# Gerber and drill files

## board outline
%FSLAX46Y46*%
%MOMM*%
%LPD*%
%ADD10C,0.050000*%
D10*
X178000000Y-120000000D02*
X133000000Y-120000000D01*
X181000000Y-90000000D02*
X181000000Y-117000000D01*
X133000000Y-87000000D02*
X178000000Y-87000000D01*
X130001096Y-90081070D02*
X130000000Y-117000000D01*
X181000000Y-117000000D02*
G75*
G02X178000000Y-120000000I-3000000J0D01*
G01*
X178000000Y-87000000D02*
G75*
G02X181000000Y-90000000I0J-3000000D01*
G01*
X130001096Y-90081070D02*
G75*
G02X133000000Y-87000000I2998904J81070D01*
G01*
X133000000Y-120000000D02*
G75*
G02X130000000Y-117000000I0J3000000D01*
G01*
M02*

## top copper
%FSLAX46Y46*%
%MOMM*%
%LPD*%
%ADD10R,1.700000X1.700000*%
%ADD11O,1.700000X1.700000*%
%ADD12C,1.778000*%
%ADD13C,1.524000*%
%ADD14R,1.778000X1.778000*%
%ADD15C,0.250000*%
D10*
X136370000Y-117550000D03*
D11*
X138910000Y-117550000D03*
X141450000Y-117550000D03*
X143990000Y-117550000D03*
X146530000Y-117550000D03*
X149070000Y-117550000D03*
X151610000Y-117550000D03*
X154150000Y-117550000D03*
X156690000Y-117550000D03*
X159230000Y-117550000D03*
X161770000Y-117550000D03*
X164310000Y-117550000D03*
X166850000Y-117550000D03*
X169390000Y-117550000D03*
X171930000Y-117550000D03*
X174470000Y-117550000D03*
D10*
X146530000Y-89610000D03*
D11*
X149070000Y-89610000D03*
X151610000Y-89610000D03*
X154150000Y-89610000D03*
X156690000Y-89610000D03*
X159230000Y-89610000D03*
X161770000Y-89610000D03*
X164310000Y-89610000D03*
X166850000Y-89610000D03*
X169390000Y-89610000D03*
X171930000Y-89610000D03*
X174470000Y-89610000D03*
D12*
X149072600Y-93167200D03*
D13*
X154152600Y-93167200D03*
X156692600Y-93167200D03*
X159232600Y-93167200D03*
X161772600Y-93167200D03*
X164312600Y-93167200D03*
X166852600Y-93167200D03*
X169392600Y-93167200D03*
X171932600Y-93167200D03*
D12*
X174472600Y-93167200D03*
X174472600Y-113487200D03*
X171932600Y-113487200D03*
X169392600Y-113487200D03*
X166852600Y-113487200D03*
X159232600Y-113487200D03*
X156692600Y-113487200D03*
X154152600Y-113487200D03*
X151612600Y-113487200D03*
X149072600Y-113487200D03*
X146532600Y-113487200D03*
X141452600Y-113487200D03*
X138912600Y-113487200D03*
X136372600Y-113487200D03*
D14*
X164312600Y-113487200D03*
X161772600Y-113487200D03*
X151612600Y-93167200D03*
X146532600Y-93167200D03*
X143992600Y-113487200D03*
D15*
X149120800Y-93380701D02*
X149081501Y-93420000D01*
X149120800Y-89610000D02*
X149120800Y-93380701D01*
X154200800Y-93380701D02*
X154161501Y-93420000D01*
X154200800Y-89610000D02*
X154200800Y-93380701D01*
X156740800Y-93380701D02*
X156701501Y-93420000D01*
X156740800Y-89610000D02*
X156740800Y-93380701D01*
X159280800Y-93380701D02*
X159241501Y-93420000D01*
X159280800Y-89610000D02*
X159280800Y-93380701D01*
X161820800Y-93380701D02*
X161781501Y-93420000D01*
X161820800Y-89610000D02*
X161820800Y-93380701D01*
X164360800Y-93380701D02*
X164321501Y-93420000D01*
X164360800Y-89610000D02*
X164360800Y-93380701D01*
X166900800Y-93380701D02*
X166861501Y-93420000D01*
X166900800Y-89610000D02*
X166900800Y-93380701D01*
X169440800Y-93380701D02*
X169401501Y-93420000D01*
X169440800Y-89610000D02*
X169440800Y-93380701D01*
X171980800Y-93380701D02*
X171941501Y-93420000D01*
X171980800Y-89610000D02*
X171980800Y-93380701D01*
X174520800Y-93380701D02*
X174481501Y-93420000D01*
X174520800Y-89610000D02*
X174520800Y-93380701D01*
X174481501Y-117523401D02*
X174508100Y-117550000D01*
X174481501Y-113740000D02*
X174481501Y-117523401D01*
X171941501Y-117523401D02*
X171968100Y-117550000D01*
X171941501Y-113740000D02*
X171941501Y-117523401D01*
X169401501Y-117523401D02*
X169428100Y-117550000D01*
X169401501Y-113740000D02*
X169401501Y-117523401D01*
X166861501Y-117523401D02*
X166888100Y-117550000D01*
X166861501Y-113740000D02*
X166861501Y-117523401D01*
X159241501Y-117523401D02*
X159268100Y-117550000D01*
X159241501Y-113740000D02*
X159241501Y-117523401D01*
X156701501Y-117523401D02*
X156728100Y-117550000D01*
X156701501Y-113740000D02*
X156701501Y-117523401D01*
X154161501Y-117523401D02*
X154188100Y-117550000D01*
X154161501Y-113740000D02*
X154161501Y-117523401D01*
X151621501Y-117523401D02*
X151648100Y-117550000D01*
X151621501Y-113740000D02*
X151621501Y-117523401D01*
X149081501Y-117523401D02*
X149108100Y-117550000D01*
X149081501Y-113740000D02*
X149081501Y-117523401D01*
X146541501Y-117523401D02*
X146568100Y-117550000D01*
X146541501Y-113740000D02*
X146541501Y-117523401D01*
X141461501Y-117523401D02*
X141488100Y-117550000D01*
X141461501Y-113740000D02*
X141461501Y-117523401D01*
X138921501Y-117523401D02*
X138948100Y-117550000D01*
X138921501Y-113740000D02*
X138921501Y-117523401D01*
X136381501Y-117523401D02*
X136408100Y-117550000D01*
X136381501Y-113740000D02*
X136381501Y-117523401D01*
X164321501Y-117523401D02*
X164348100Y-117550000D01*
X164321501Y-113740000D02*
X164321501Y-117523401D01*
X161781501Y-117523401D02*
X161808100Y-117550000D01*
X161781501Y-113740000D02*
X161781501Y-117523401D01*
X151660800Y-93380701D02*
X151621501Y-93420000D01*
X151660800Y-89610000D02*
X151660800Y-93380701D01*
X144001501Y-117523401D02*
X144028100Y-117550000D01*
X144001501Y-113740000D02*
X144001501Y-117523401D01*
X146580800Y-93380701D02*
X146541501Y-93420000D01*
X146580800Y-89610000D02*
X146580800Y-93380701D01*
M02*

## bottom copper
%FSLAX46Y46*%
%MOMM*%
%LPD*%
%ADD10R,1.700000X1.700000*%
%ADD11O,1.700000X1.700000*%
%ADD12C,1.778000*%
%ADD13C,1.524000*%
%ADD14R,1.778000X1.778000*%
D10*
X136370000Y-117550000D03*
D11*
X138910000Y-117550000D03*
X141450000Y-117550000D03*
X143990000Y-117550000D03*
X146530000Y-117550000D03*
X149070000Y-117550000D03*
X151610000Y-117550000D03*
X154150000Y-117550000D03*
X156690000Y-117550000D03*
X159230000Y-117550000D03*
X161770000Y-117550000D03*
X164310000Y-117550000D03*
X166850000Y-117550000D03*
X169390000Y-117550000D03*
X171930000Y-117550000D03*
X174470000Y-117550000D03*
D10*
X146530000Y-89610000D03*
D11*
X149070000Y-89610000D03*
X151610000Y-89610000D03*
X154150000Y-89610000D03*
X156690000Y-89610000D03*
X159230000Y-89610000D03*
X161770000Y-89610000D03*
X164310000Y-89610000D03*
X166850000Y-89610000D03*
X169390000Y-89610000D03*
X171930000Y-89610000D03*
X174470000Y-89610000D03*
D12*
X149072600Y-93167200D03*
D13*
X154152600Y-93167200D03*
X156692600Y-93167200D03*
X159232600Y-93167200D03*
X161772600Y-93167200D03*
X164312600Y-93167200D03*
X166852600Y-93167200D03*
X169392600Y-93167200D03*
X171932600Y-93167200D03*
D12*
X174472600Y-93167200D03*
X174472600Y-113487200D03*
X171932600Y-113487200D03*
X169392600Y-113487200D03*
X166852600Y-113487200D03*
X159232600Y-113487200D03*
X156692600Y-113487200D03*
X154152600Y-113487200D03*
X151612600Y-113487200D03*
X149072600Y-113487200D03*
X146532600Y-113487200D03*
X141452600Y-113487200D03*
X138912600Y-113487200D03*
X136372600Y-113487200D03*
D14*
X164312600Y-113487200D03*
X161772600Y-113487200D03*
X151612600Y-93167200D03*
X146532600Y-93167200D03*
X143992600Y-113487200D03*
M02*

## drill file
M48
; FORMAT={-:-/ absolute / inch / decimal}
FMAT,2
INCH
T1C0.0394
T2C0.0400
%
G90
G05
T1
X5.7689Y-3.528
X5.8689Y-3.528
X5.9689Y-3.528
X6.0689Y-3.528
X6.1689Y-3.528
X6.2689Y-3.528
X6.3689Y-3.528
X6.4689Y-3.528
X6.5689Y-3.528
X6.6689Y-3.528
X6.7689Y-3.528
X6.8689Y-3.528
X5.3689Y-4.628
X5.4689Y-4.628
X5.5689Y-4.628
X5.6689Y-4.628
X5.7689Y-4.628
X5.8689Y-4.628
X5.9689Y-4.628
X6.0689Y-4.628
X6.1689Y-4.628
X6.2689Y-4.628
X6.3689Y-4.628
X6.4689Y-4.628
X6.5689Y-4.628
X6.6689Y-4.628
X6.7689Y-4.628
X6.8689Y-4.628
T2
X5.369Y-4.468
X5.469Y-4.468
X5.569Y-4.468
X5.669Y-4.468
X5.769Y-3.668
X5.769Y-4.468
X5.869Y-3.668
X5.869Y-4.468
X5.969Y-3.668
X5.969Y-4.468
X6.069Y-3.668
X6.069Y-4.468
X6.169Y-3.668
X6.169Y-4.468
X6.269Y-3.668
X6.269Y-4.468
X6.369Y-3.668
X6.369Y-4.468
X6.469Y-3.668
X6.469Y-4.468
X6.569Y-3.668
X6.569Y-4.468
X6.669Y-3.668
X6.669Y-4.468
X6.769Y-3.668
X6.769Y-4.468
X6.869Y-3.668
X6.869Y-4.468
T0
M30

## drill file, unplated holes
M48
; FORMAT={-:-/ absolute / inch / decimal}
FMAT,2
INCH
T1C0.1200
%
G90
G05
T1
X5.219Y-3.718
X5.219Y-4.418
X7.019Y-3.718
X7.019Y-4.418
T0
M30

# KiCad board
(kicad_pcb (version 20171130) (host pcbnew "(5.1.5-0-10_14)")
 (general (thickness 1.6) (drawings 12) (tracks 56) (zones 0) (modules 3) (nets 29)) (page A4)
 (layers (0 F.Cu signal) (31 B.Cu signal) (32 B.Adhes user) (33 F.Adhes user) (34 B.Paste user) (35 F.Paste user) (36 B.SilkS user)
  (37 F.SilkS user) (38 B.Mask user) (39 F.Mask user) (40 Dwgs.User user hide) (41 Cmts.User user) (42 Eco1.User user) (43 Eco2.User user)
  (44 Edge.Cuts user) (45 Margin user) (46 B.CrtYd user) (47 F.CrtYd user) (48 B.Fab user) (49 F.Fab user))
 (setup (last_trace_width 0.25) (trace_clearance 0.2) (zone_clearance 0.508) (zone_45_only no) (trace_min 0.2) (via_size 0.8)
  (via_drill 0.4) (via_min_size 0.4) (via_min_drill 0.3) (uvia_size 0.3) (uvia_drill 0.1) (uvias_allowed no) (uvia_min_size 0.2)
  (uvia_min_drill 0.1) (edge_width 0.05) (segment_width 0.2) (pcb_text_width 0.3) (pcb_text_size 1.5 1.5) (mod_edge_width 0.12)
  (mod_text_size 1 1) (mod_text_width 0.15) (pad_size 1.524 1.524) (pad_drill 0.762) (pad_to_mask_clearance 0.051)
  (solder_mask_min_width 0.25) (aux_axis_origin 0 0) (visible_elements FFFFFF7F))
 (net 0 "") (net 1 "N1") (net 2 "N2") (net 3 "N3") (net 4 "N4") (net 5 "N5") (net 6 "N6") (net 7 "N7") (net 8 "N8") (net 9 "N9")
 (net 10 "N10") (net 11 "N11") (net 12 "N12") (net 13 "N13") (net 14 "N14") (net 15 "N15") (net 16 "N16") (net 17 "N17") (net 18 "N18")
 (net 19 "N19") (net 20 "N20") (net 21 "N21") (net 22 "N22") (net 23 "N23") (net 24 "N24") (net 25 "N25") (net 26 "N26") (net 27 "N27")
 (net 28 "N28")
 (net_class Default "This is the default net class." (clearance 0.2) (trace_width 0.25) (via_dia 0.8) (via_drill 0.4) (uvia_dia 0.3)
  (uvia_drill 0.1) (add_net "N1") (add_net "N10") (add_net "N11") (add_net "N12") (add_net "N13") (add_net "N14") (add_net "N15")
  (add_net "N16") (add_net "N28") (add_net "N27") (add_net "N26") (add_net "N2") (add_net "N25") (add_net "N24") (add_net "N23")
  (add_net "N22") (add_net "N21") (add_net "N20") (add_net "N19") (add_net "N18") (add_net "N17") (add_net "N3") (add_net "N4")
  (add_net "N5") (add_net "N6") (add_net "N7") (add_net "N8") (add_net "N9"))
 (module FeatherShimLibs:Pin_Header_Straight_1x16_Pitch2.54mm (layer F.Cu) (at 136.37 117.55 90)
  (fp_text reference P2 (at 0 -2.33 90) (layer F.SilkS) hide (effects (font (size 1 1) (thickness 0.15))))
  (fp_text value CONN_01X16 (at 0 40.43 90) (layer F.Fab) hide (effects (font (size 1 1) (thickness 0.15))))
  (pad 1 thru_hole rect (at 0 0 90) (size 1.7 1.7) (drill 1) (layers *.Cu *.Mask) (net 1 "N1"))
  (pad 2 thru_hole oval (at 0 2.54 90) (size 1.7 1.7) (drill 1) (layers *.Cu *.Mask) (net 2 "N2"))
  (pad 3 thru_hole oval (at 0 5.08 90) (size 1.7 1.7) (drill 1) (layers *.Cu *.Mask) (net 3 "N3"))
  (pad 4 thru_hole oval (at 0 7.62 90) (size 1.7 1.7) (drill 1) (layers *.Cu *.Mask) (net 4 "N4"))
  (pad 5 thru_hole oval (at 0 10.16 90) (size 1.7 1.7) (drill 1) (layers *.Cu *.Mask) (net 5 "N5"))
  (pad 6 thru_hole oval (at 0 12.7 90) (size 1.7 1.7) (drill 1) (layers *.Cu *.Mask) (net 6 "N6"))
  (pad 7 thru_hole oval (at 0 15.24 90) (size 1.7 1.7) (drill 1) (layers *.Cu *.Mask) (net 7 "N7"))
  (pad 8 thru_hole oval (at 0 17.78 90) (size 1.7 1.7) (drill 1) (layers *.Cu *.Mask) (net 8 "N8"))
  (pad 9 thru_hole oval (at 0 20.32 90) (size 1.7 1.7) (drill 1) (layers *.Cu *.Mask) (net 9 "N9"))
  (pad 10 thru_hole oval (at 0 22.86 90) (size 1.7 1.7) (drill 1) (layers *.Cu *.Mask) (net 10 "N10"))
  (pad 11 thru_hole oval (at 0 25.4 90) (size 1.7 1.7) (drill 1) (layers *.Cu *.Mask) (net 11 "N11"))
  (pad 12 thru_hole oval (at 0 27.94 90) (size 1.7 1.7) (drill 1) (layers *.Cu *.Mask) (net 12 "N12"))
  (pad 13 thru_hole oval (at 0 30.48 90) (size 1.7 1.7) (drill 1) (layers *.Cu *.Mask) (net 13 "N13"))
  (pad 14 thru_hole oval (at 0 33.02 90) (size 1.7 1.7) (drill 1) (layers *.Cu *.Mask) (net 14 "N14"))
  (pad 15 thru_hole oval (at 0 35.56 90) (size 1.7 1.7) (drill 1) (layers *.Cu *.Mask) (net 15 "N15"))
  (pad 16 thru_hole oval (at 0 38.1 90) (size 1.7 1.7) (drill 1) (layers *.Cu *.Mask) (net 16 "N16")))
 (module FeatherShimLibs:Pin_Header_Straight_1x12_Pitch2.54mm (layer F.Cu) (at 146.53 89.61 90)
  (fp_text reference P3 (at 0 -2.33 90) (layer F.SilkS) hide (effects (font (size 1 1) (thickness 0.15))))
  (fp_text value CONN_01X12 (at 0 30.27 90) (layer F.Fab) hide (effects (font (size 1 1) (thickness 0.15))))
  (pad 1 thru_hole rect (at 0 0 90) (size 1.7 1.7) (drill 1) (layers *.Cu *.Mask) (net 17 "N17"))
  (pad 2 thru_hole oval (at 0 2.54 90) (size 1.7 1.7) (drill 1) (layers *.Cu *.Mask) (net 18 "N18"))
  (pad 3 thru_hole oval (at 0 5.08 90) (size 1.7 1.7) (drill 1) (layers *.Cu *.Mask) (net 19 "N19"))
  (pad 4 thru_hole oval (at 0 7.62 90) (size 1.7 1.7) (drill 1) (layers *.Cu *.Mask) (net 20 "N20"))
  (pad 5 thru_hole oval (at 0 10.16 90) (size 1.7 1.7) (drill 1) (layers *.Cu *.Mask) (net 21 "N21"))
  (pad 6 thru_hole oval (at 0 12.7 90) (size 1.7 1.7) (drill 1) (layers *.Cu *.Mask) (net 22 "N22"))
  (pad 7 thru_hole oval (at 0 15.24 90) (size 1.7 1.7) (drill 1) (layers *.Cu *.Mask) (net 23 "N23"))
  (pad 8 thru_hole oval (at 0 17.78 90) (size 1.7 1.7) (drill 1) (layers *.Cu *.Mask) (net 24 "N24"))
  (pad 9 thru_hole oval (at 0 20.32 90) (size 1.7 1.7) (drill 1) (layers *.Cu *.Mask) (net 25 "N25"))
  (pad 10 thru_hole oval (at 0 22.86 90) (size 1.7 1.7) (drill 1) (layers *.Cu *.Mask) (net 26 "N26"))
  (pad 11 thru_hole oval (at 0 25.4 90) (size 1.7 1.7) (drill 1) (layers *.Cu *.Mask) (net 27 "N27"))
  (pad 12 thru_hole oval (at 0 27.94 90) (size 1.7 1.7) (drill 1) (layers *.Cu *.Mask) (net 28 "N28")))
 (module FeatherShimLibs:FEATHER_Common (layer F.Cu) (at 155.4226 103.3272)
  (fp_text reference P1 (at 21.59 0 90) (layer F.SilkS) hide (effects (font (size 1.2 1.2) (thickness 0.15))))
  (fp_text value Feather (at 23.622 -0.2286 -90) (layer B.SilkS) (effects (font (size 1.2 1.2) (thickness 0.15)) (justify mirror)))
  (pad "" np_thru_hole circle (at -22.86 -8.89) (size 3.048 3.048) (drill 3.048) (layers *.Cu *.Mask))
  (pad "" np_thru_hole circle (at 22.86 -8.89) (size 3.048 3.048) (drill 3.048) (layers *.Cu *.Mask))
  (pad "" np_thru_hole circle (at 22.86 8.89) (size 3.048 3.048) (drill 3.048) (layers *.Cu *.Mask))
  (pad "" np_thru_hole circle (at -22.86 8.89) (size 3.048 3.048) (drill 3.048) (layers *.Cu *.Mask))
  (pad 27 thru_hole circle (at -6.35 -10.16) (size 1.778 1.778) (drill 1.016) (layers *.Cu *.Mask) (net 18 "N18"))
  (pad 25 thru_hole circle (at -1.27 -10.16) (size 1.524 1.524) (drill 1.016) (layers *.Cu *.Mask) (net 20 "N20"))
  (pad 24 thru_hole circle (at 1.27 -10.16) (size 1.524 1.524) (drill 1.016) (layers *.Cu *.Mask) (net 21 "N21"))
  (pad 23 thru_hole circle (at 3.81 -10.16) (size 1.524 1.524) (drill 1.016) (layers *.Cu *.Mask) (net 22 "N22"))
  (pad 22 thru_hole circle (at 6.35 -10.16) (size 1.524 1.524) (drill 1.016) (layers *.Cu *.Mask) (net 23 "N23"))
  (pad 21 thru_hole circle (at 8.89 -10.16) (size 1.524 1.524) (drill 1.016) (layers *.Cu *.Mask) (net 24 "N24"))
  (pad 20 thru_hole circle (at 11.43 -10.16) (size 1.524 1.524) (drill 1.016) (layers *.Cu *.Mask) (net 25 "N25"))
  (pad 19 thru_hole circle (at 13.97 -10.16) (size 1.524 1.524) (drill 1.016) (layers *.Cu *.Mask) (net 26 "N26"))
  (pad 18 thru_hole circle (at 16.51 -10.16) (size 1.524 1.524) (drill 1.016) (layers *.Cu *.Mask) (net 27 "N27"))
  (pad 17 thru_hole circle (at 19.05 -10.16) (size 1.778 1.778) (drill 1.016) (layers *.Cu *.Mask) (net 28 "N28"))
  (pad 16 thru_hole circle (at 19.05 10.16) (size 1.778 1.778) (drill 1.016) (layers *.Cu *.Mask) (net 16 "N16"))
  (pad 15 thru_hole circle (at 16.51 10.16) (size 1.778 1.778) (drill 1.016) (layers *.Cu *.Mask) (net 15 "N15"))
  (pad 14 thru_hole circle (at 13.97 10.16) (size 1.778 1.778) (drill 1.016) (layers *.Cu *.Mask) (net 14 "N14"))
  (pad 13 thru_hole circle (at 11.43 10.16) (size 1.778 1.778) (drill 1.016) (layers *.Cu *.Mask) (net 13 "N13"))
  (pad 10 thru_hole circle (at 3.81 10.16) (size 1.778 1.778) (drill 1.016) (layers *.Cu *.Mask) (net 10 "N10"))
  (pad 9 thru_hole circle (at 1.27 10.16) (size 1.778 1.778) (drill 1.016) (layers *.Cu *.Mask) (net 9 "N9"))
  (pad 8 thru_hole circle (at -1.27 10.16) (size 1.778 1.778) (drill 1.016) (layers *.Cu *.Mask) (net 8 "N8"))
  (pad 7 thru_hole circle (at -3.81 10.16) (size 1.778 1.778) (drill 1.016) (layers *.Cu *.Mask) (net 7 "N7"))
  (pad 6 thru_hole circle (at -6.35 10.16) (size 1.778 1.778) (drill 1.016) (layers *.Cu *.Mask) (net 6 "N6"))
  (pad 5 thru_hole circle (at -8.89 10.16) (size 1.778 1.778) (drill 1.016) (layers *.Cu *.Mask) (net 5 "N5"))
  (pad 3 thru_hole circle (at -13.97 10.16) (size 1.778 1.778) (drill 1.016) (layers *.Cu *.Mask) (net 3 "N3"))
  (pad 2 thru_hole circle (at -16.51 10.16) (size 1.778 1.778) (drill 1.016) (layers *.Cu *.Mask) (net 2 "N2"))
  (pad 1 thru_hole circle (at -19.05 10.16) (size 1.778 1.778) (drill 1.016) (layers *.Cu *.Mask) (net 1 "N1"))
  (pad 12 thru_hole rect (at 8.89 10.16) (size 1.778 1.778) (drill 1.016) (layers *.Cu *.Mask) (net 12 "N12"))
  (pad 11 thru_hole rect (at 6.35 10.16) (size 1.778 1.778) (drill 1.016) (layers *.Cu *.Mask) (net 11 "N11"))
  (pad 26 thru_hole rect (at -3.81 -10.16) (size 1.778 1.778) (drill 1.016) (layers *.Cu *.Mask) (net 19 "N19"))
  (pad 28 thru_hole rect (at -8.89 -10.16) (size 1.778 1.778) (drill 1.016) (layers *.Cu *.Mask) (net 17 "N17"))
  (pad 4 thru_hole rect (at -11.43 10.16) (size 1.778 1.778) (drill 1.016) (layers *.Cu *.Mask) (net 4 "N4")))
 (gr_line (start 178 120) (end 133 120) (layer Edge.Cuts) (width 0.05))
 (gr_line (start 181 90) (end 181 117) (layer Edge.Cuts) (width 0.05))
 (gr_line (start 133 87) (end 178 87) (layer Edge.Cuts) (width 0.05))
 (gr_line (start 130.001096 90.08107) (end 130 117) (layer Edge.Cuts) (width 0.05))
 (gr_arc (start 178 117) (end 178 120) (angle -90) (layer Edge.Cuts) (width 0.05))
 (gr_arc (start 178 90) (end 181 90) (angle -90) (layer Edge.Cuts) (width 0.05))
 (gr_arc (start 133 90) (end 133 87) (angle -91.54851876) (layer Edge.Cuts) (width 0.05))
 (gr_arc (start 133 117) (end 130 117) (angle -90) (layer Edge.Cuts) (width 0.05))
 (segment (start 149.1208 93.380701) (end 149.081501 93.42) (width 0.25) (layer F.Cu) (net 18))
 (segment (start 149.1208 89.61) (end 149.1208 93.380701) (width 0.25) (layer F.Cu) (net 18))
 (segment (start 154.2008 93.380701) (end 154.161501 93.42) (width 0.25) (layer F.Cu) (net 20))
 (segment (start 154.2008 89.61) (end 154.2008 93.380701) (width 0.25) (layer F.Cu) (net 20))
 (segment (start 156.7408 93.380701) (end 156.701501 93.42) (width 0.25) (layer F.Cu) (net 21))
 (segment (start 156.7408 89.61) (end 156.7408 93.380701) (width 0.25) (layer F.Cu) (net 21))
 (segment (start 159.2808 93.380701) (end 159.241501 93.42) (width 0.25) (layer F.Cu) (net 22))
 (segment (start 159.2808 89.61) (end 159.2808 93.380701) (width 0.25) (layer F.Cu) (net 22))
 (segment (start 161.8208 93.380701) (end 161.781501 93.42) (width 0.25) (layer F.Cu) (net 23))
 (segment (start 161.8208 89.61) (end 161.8208 93.380701) (width 0.25) (layer F.Cu) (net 23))
 (segment (start 164.3608 93.380701) (end 164.321501 93.42) (width 0.25) (layer F.Cu) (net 24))
 (segment (start 164.3608 89.61) (end 164.3608 93.380701) (width 0.25) (layer F.Cu) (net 24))
 (segment (start 166.9008 93.380701) (end 166.861501 93.42) (width 0.25) (layer F.Cu) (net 25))
 (segment (start 166.9008 89.61) (end 166.9008 93.380701) (width 0.25) (layer F.Cu) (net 25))
 (segment (start 169.4408 93.380701) (end 169.401501 93.42) (width 0.25) (layer F.Cu) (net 26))
 (segment (start 169.4408 89.61) (end 169.4408 93.380701) (width 0.25) (layer F.Cu) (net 26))
 (segment (start 171.9808 93.380701) (end 171.941501 93.42) (width 0.25) (layer F.Cu) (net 27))
 (segment (start 171.9808 89.61) (end 171.9808 93.380701) (width 0.25) (layer F.Cu) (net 27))
 (segment (start 174.5208 93.380701) (end 174.481501 93.42) (width 0.25) (layer F.Cu) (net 28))
 (segment (start 174.5208 89.61) (end 174.5208 93.380701) (width 0.25) (layer F.Cu) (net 28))
 (segment (start 174.481501 117.523401) (end 174.5081 117.55) (width 0.25) (layer F.Cu) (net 16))
 (segment (start 174.481501 113.74) (end 174.481501 117.523401) (width 0.25) (layer F.Cu) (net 16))
 (segment (start 171.941501 117.523401) (end 171.9681 117.55) (width 0.25) (layer F.Cu) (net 15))
 (segment (start 171.941501 113.74) (end 171.941501 117.523401) (width 0.25) (layer F.Cu) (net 15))
 (segment (start 169.401501 117.523401) (end 169.4281 117.55) (width 0.25) (layer F.Cu) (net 14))
 (segment (start 169.401501 113.74) (end 169.401501 117.523401) (width 0.25) (layer F.Cu) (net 14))
 (segment (start 166.861501 117.523401) (end 166.8881 117.55) (width 0.25) (layer F.Cu) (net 13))
 (segment (start 166.861501 113.74) (end 166.861501 117.523401) (width 0.25) (layer F.Cu) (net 13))
 (segment (start 159.241501 117.523401) (end 159.2681 117.55) (width 0.25) (layer F.Cu) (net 10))
 (segment (start 159.241501 113.74) (end 159.241501 117.523401) (width 0.25) (layer F.Cu) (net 10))
 (segment (start 156.701501 117.523401) (end 156.7281 117.55) (width 0.25) (layer F.Cu) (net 9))
 (segment (start 156.701501 113.74) (end 156.701501 117.523401) (width 0.25) (layer F.Cu) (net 9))
 (segment (start 154.161501 117.523401) (end 154.1881 117.55) (width 0.25) (layer F.Cu) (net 8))
 (segment (start 154.161501 113.74) (end 154.161501 117.523401) (width 0.25) (layer F.Cu) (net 8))
 (segment (start 151.621501 117.523401) (end 151.6481 117.55) (width 0.25) (layer F.Cu) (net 7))
 (segment (start 151.621501 113.74) (end 151.621501 117.523401) (width 0.25) (layer F.Cu) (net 7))
 (segment (start 149.081501 117.523401) (end 149.1081 117.55) (width 0.25) (layer F.Cu) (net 6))
 (segment (start 149.081501 113.74) (end 149.081501 117.523401) (width 0.25) (layer F.Cu) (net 6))
 (segment (start 146.541501 117.523401) (end 146.5681 117.55) (width 0.25) (layer F.Cu) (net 5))
 (segment (start 146.541501 113.74) (end 146.541501 117.523401) (width 0.25) (layer F.Cu) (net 5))
 (segment (start 141.461501 117.523401) (end 141.4881 117.55) (width 0.25) (layer F.Cu) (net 3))
 (segment (start 141.461501 113.74) (end 141.461501 117.523401) (width 0.25) (layer F.Cu) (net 3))
 (segment (start 138.921501 117.523401) (end 138.9481 117.55) (width 0.25) (layer F.Cu) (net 2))
 (segment (start 138.921501 113.74) (end 138.921501 117.523401) (width 0.25) (layer F.Cu) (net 2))
 (segment (start 136.381501 117.523401) (end 136.4081 117.55) (width 0.25) (layer F.Cu) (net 1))
 (segment (start 136.381501 113.74) (end 136.381501 117.523401) (width 0.25) (layer F.Cu) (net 1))
 (segment (start 164.321501 117.523401) (end 164.3481 117.55) (width 0.25) (layer F.Cu) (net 12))
 (segment (start 164.321501 113.74) (end 164.321501 117.523401) (width 0.25) (layer F.Cu) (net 12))
 (segment (start 161.781501 117.523401) (end 161.8081 117.55) (width 0.25) (layer F.Cu) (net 11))
 (segment (start 161.781501 113.74) (end 161.781501 117.523401) (width 0.25) (layer F.Cu) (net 11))
 (segment (start 151.6608 93.380701) (end 151.621501 93.42) (width 0.25) (layer F.Cu) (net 19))
 (segment (start 151.6608 89.61) (end 151.6608 93.380701) (width 0.25) (layer F.Cu) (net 19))
 (segment (start 144.001501 117.523401) (end 144.0281 117.55) (width 0.25) (layer F.Cu) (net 4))
 (segment (start 144.001501 113.74) (end 144.001501 117.523401) (width 0.25) (layer F.Cu) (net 4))
 (segment (start 146.5808 93.380701) (end 146.541501 93.42) (width 0.25) (layer F.Cu) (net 17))
 (segment (start 146.5808 89.61) (end 146.5808 93.380701) (width 0.25) (layer F.Cu) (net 17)))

